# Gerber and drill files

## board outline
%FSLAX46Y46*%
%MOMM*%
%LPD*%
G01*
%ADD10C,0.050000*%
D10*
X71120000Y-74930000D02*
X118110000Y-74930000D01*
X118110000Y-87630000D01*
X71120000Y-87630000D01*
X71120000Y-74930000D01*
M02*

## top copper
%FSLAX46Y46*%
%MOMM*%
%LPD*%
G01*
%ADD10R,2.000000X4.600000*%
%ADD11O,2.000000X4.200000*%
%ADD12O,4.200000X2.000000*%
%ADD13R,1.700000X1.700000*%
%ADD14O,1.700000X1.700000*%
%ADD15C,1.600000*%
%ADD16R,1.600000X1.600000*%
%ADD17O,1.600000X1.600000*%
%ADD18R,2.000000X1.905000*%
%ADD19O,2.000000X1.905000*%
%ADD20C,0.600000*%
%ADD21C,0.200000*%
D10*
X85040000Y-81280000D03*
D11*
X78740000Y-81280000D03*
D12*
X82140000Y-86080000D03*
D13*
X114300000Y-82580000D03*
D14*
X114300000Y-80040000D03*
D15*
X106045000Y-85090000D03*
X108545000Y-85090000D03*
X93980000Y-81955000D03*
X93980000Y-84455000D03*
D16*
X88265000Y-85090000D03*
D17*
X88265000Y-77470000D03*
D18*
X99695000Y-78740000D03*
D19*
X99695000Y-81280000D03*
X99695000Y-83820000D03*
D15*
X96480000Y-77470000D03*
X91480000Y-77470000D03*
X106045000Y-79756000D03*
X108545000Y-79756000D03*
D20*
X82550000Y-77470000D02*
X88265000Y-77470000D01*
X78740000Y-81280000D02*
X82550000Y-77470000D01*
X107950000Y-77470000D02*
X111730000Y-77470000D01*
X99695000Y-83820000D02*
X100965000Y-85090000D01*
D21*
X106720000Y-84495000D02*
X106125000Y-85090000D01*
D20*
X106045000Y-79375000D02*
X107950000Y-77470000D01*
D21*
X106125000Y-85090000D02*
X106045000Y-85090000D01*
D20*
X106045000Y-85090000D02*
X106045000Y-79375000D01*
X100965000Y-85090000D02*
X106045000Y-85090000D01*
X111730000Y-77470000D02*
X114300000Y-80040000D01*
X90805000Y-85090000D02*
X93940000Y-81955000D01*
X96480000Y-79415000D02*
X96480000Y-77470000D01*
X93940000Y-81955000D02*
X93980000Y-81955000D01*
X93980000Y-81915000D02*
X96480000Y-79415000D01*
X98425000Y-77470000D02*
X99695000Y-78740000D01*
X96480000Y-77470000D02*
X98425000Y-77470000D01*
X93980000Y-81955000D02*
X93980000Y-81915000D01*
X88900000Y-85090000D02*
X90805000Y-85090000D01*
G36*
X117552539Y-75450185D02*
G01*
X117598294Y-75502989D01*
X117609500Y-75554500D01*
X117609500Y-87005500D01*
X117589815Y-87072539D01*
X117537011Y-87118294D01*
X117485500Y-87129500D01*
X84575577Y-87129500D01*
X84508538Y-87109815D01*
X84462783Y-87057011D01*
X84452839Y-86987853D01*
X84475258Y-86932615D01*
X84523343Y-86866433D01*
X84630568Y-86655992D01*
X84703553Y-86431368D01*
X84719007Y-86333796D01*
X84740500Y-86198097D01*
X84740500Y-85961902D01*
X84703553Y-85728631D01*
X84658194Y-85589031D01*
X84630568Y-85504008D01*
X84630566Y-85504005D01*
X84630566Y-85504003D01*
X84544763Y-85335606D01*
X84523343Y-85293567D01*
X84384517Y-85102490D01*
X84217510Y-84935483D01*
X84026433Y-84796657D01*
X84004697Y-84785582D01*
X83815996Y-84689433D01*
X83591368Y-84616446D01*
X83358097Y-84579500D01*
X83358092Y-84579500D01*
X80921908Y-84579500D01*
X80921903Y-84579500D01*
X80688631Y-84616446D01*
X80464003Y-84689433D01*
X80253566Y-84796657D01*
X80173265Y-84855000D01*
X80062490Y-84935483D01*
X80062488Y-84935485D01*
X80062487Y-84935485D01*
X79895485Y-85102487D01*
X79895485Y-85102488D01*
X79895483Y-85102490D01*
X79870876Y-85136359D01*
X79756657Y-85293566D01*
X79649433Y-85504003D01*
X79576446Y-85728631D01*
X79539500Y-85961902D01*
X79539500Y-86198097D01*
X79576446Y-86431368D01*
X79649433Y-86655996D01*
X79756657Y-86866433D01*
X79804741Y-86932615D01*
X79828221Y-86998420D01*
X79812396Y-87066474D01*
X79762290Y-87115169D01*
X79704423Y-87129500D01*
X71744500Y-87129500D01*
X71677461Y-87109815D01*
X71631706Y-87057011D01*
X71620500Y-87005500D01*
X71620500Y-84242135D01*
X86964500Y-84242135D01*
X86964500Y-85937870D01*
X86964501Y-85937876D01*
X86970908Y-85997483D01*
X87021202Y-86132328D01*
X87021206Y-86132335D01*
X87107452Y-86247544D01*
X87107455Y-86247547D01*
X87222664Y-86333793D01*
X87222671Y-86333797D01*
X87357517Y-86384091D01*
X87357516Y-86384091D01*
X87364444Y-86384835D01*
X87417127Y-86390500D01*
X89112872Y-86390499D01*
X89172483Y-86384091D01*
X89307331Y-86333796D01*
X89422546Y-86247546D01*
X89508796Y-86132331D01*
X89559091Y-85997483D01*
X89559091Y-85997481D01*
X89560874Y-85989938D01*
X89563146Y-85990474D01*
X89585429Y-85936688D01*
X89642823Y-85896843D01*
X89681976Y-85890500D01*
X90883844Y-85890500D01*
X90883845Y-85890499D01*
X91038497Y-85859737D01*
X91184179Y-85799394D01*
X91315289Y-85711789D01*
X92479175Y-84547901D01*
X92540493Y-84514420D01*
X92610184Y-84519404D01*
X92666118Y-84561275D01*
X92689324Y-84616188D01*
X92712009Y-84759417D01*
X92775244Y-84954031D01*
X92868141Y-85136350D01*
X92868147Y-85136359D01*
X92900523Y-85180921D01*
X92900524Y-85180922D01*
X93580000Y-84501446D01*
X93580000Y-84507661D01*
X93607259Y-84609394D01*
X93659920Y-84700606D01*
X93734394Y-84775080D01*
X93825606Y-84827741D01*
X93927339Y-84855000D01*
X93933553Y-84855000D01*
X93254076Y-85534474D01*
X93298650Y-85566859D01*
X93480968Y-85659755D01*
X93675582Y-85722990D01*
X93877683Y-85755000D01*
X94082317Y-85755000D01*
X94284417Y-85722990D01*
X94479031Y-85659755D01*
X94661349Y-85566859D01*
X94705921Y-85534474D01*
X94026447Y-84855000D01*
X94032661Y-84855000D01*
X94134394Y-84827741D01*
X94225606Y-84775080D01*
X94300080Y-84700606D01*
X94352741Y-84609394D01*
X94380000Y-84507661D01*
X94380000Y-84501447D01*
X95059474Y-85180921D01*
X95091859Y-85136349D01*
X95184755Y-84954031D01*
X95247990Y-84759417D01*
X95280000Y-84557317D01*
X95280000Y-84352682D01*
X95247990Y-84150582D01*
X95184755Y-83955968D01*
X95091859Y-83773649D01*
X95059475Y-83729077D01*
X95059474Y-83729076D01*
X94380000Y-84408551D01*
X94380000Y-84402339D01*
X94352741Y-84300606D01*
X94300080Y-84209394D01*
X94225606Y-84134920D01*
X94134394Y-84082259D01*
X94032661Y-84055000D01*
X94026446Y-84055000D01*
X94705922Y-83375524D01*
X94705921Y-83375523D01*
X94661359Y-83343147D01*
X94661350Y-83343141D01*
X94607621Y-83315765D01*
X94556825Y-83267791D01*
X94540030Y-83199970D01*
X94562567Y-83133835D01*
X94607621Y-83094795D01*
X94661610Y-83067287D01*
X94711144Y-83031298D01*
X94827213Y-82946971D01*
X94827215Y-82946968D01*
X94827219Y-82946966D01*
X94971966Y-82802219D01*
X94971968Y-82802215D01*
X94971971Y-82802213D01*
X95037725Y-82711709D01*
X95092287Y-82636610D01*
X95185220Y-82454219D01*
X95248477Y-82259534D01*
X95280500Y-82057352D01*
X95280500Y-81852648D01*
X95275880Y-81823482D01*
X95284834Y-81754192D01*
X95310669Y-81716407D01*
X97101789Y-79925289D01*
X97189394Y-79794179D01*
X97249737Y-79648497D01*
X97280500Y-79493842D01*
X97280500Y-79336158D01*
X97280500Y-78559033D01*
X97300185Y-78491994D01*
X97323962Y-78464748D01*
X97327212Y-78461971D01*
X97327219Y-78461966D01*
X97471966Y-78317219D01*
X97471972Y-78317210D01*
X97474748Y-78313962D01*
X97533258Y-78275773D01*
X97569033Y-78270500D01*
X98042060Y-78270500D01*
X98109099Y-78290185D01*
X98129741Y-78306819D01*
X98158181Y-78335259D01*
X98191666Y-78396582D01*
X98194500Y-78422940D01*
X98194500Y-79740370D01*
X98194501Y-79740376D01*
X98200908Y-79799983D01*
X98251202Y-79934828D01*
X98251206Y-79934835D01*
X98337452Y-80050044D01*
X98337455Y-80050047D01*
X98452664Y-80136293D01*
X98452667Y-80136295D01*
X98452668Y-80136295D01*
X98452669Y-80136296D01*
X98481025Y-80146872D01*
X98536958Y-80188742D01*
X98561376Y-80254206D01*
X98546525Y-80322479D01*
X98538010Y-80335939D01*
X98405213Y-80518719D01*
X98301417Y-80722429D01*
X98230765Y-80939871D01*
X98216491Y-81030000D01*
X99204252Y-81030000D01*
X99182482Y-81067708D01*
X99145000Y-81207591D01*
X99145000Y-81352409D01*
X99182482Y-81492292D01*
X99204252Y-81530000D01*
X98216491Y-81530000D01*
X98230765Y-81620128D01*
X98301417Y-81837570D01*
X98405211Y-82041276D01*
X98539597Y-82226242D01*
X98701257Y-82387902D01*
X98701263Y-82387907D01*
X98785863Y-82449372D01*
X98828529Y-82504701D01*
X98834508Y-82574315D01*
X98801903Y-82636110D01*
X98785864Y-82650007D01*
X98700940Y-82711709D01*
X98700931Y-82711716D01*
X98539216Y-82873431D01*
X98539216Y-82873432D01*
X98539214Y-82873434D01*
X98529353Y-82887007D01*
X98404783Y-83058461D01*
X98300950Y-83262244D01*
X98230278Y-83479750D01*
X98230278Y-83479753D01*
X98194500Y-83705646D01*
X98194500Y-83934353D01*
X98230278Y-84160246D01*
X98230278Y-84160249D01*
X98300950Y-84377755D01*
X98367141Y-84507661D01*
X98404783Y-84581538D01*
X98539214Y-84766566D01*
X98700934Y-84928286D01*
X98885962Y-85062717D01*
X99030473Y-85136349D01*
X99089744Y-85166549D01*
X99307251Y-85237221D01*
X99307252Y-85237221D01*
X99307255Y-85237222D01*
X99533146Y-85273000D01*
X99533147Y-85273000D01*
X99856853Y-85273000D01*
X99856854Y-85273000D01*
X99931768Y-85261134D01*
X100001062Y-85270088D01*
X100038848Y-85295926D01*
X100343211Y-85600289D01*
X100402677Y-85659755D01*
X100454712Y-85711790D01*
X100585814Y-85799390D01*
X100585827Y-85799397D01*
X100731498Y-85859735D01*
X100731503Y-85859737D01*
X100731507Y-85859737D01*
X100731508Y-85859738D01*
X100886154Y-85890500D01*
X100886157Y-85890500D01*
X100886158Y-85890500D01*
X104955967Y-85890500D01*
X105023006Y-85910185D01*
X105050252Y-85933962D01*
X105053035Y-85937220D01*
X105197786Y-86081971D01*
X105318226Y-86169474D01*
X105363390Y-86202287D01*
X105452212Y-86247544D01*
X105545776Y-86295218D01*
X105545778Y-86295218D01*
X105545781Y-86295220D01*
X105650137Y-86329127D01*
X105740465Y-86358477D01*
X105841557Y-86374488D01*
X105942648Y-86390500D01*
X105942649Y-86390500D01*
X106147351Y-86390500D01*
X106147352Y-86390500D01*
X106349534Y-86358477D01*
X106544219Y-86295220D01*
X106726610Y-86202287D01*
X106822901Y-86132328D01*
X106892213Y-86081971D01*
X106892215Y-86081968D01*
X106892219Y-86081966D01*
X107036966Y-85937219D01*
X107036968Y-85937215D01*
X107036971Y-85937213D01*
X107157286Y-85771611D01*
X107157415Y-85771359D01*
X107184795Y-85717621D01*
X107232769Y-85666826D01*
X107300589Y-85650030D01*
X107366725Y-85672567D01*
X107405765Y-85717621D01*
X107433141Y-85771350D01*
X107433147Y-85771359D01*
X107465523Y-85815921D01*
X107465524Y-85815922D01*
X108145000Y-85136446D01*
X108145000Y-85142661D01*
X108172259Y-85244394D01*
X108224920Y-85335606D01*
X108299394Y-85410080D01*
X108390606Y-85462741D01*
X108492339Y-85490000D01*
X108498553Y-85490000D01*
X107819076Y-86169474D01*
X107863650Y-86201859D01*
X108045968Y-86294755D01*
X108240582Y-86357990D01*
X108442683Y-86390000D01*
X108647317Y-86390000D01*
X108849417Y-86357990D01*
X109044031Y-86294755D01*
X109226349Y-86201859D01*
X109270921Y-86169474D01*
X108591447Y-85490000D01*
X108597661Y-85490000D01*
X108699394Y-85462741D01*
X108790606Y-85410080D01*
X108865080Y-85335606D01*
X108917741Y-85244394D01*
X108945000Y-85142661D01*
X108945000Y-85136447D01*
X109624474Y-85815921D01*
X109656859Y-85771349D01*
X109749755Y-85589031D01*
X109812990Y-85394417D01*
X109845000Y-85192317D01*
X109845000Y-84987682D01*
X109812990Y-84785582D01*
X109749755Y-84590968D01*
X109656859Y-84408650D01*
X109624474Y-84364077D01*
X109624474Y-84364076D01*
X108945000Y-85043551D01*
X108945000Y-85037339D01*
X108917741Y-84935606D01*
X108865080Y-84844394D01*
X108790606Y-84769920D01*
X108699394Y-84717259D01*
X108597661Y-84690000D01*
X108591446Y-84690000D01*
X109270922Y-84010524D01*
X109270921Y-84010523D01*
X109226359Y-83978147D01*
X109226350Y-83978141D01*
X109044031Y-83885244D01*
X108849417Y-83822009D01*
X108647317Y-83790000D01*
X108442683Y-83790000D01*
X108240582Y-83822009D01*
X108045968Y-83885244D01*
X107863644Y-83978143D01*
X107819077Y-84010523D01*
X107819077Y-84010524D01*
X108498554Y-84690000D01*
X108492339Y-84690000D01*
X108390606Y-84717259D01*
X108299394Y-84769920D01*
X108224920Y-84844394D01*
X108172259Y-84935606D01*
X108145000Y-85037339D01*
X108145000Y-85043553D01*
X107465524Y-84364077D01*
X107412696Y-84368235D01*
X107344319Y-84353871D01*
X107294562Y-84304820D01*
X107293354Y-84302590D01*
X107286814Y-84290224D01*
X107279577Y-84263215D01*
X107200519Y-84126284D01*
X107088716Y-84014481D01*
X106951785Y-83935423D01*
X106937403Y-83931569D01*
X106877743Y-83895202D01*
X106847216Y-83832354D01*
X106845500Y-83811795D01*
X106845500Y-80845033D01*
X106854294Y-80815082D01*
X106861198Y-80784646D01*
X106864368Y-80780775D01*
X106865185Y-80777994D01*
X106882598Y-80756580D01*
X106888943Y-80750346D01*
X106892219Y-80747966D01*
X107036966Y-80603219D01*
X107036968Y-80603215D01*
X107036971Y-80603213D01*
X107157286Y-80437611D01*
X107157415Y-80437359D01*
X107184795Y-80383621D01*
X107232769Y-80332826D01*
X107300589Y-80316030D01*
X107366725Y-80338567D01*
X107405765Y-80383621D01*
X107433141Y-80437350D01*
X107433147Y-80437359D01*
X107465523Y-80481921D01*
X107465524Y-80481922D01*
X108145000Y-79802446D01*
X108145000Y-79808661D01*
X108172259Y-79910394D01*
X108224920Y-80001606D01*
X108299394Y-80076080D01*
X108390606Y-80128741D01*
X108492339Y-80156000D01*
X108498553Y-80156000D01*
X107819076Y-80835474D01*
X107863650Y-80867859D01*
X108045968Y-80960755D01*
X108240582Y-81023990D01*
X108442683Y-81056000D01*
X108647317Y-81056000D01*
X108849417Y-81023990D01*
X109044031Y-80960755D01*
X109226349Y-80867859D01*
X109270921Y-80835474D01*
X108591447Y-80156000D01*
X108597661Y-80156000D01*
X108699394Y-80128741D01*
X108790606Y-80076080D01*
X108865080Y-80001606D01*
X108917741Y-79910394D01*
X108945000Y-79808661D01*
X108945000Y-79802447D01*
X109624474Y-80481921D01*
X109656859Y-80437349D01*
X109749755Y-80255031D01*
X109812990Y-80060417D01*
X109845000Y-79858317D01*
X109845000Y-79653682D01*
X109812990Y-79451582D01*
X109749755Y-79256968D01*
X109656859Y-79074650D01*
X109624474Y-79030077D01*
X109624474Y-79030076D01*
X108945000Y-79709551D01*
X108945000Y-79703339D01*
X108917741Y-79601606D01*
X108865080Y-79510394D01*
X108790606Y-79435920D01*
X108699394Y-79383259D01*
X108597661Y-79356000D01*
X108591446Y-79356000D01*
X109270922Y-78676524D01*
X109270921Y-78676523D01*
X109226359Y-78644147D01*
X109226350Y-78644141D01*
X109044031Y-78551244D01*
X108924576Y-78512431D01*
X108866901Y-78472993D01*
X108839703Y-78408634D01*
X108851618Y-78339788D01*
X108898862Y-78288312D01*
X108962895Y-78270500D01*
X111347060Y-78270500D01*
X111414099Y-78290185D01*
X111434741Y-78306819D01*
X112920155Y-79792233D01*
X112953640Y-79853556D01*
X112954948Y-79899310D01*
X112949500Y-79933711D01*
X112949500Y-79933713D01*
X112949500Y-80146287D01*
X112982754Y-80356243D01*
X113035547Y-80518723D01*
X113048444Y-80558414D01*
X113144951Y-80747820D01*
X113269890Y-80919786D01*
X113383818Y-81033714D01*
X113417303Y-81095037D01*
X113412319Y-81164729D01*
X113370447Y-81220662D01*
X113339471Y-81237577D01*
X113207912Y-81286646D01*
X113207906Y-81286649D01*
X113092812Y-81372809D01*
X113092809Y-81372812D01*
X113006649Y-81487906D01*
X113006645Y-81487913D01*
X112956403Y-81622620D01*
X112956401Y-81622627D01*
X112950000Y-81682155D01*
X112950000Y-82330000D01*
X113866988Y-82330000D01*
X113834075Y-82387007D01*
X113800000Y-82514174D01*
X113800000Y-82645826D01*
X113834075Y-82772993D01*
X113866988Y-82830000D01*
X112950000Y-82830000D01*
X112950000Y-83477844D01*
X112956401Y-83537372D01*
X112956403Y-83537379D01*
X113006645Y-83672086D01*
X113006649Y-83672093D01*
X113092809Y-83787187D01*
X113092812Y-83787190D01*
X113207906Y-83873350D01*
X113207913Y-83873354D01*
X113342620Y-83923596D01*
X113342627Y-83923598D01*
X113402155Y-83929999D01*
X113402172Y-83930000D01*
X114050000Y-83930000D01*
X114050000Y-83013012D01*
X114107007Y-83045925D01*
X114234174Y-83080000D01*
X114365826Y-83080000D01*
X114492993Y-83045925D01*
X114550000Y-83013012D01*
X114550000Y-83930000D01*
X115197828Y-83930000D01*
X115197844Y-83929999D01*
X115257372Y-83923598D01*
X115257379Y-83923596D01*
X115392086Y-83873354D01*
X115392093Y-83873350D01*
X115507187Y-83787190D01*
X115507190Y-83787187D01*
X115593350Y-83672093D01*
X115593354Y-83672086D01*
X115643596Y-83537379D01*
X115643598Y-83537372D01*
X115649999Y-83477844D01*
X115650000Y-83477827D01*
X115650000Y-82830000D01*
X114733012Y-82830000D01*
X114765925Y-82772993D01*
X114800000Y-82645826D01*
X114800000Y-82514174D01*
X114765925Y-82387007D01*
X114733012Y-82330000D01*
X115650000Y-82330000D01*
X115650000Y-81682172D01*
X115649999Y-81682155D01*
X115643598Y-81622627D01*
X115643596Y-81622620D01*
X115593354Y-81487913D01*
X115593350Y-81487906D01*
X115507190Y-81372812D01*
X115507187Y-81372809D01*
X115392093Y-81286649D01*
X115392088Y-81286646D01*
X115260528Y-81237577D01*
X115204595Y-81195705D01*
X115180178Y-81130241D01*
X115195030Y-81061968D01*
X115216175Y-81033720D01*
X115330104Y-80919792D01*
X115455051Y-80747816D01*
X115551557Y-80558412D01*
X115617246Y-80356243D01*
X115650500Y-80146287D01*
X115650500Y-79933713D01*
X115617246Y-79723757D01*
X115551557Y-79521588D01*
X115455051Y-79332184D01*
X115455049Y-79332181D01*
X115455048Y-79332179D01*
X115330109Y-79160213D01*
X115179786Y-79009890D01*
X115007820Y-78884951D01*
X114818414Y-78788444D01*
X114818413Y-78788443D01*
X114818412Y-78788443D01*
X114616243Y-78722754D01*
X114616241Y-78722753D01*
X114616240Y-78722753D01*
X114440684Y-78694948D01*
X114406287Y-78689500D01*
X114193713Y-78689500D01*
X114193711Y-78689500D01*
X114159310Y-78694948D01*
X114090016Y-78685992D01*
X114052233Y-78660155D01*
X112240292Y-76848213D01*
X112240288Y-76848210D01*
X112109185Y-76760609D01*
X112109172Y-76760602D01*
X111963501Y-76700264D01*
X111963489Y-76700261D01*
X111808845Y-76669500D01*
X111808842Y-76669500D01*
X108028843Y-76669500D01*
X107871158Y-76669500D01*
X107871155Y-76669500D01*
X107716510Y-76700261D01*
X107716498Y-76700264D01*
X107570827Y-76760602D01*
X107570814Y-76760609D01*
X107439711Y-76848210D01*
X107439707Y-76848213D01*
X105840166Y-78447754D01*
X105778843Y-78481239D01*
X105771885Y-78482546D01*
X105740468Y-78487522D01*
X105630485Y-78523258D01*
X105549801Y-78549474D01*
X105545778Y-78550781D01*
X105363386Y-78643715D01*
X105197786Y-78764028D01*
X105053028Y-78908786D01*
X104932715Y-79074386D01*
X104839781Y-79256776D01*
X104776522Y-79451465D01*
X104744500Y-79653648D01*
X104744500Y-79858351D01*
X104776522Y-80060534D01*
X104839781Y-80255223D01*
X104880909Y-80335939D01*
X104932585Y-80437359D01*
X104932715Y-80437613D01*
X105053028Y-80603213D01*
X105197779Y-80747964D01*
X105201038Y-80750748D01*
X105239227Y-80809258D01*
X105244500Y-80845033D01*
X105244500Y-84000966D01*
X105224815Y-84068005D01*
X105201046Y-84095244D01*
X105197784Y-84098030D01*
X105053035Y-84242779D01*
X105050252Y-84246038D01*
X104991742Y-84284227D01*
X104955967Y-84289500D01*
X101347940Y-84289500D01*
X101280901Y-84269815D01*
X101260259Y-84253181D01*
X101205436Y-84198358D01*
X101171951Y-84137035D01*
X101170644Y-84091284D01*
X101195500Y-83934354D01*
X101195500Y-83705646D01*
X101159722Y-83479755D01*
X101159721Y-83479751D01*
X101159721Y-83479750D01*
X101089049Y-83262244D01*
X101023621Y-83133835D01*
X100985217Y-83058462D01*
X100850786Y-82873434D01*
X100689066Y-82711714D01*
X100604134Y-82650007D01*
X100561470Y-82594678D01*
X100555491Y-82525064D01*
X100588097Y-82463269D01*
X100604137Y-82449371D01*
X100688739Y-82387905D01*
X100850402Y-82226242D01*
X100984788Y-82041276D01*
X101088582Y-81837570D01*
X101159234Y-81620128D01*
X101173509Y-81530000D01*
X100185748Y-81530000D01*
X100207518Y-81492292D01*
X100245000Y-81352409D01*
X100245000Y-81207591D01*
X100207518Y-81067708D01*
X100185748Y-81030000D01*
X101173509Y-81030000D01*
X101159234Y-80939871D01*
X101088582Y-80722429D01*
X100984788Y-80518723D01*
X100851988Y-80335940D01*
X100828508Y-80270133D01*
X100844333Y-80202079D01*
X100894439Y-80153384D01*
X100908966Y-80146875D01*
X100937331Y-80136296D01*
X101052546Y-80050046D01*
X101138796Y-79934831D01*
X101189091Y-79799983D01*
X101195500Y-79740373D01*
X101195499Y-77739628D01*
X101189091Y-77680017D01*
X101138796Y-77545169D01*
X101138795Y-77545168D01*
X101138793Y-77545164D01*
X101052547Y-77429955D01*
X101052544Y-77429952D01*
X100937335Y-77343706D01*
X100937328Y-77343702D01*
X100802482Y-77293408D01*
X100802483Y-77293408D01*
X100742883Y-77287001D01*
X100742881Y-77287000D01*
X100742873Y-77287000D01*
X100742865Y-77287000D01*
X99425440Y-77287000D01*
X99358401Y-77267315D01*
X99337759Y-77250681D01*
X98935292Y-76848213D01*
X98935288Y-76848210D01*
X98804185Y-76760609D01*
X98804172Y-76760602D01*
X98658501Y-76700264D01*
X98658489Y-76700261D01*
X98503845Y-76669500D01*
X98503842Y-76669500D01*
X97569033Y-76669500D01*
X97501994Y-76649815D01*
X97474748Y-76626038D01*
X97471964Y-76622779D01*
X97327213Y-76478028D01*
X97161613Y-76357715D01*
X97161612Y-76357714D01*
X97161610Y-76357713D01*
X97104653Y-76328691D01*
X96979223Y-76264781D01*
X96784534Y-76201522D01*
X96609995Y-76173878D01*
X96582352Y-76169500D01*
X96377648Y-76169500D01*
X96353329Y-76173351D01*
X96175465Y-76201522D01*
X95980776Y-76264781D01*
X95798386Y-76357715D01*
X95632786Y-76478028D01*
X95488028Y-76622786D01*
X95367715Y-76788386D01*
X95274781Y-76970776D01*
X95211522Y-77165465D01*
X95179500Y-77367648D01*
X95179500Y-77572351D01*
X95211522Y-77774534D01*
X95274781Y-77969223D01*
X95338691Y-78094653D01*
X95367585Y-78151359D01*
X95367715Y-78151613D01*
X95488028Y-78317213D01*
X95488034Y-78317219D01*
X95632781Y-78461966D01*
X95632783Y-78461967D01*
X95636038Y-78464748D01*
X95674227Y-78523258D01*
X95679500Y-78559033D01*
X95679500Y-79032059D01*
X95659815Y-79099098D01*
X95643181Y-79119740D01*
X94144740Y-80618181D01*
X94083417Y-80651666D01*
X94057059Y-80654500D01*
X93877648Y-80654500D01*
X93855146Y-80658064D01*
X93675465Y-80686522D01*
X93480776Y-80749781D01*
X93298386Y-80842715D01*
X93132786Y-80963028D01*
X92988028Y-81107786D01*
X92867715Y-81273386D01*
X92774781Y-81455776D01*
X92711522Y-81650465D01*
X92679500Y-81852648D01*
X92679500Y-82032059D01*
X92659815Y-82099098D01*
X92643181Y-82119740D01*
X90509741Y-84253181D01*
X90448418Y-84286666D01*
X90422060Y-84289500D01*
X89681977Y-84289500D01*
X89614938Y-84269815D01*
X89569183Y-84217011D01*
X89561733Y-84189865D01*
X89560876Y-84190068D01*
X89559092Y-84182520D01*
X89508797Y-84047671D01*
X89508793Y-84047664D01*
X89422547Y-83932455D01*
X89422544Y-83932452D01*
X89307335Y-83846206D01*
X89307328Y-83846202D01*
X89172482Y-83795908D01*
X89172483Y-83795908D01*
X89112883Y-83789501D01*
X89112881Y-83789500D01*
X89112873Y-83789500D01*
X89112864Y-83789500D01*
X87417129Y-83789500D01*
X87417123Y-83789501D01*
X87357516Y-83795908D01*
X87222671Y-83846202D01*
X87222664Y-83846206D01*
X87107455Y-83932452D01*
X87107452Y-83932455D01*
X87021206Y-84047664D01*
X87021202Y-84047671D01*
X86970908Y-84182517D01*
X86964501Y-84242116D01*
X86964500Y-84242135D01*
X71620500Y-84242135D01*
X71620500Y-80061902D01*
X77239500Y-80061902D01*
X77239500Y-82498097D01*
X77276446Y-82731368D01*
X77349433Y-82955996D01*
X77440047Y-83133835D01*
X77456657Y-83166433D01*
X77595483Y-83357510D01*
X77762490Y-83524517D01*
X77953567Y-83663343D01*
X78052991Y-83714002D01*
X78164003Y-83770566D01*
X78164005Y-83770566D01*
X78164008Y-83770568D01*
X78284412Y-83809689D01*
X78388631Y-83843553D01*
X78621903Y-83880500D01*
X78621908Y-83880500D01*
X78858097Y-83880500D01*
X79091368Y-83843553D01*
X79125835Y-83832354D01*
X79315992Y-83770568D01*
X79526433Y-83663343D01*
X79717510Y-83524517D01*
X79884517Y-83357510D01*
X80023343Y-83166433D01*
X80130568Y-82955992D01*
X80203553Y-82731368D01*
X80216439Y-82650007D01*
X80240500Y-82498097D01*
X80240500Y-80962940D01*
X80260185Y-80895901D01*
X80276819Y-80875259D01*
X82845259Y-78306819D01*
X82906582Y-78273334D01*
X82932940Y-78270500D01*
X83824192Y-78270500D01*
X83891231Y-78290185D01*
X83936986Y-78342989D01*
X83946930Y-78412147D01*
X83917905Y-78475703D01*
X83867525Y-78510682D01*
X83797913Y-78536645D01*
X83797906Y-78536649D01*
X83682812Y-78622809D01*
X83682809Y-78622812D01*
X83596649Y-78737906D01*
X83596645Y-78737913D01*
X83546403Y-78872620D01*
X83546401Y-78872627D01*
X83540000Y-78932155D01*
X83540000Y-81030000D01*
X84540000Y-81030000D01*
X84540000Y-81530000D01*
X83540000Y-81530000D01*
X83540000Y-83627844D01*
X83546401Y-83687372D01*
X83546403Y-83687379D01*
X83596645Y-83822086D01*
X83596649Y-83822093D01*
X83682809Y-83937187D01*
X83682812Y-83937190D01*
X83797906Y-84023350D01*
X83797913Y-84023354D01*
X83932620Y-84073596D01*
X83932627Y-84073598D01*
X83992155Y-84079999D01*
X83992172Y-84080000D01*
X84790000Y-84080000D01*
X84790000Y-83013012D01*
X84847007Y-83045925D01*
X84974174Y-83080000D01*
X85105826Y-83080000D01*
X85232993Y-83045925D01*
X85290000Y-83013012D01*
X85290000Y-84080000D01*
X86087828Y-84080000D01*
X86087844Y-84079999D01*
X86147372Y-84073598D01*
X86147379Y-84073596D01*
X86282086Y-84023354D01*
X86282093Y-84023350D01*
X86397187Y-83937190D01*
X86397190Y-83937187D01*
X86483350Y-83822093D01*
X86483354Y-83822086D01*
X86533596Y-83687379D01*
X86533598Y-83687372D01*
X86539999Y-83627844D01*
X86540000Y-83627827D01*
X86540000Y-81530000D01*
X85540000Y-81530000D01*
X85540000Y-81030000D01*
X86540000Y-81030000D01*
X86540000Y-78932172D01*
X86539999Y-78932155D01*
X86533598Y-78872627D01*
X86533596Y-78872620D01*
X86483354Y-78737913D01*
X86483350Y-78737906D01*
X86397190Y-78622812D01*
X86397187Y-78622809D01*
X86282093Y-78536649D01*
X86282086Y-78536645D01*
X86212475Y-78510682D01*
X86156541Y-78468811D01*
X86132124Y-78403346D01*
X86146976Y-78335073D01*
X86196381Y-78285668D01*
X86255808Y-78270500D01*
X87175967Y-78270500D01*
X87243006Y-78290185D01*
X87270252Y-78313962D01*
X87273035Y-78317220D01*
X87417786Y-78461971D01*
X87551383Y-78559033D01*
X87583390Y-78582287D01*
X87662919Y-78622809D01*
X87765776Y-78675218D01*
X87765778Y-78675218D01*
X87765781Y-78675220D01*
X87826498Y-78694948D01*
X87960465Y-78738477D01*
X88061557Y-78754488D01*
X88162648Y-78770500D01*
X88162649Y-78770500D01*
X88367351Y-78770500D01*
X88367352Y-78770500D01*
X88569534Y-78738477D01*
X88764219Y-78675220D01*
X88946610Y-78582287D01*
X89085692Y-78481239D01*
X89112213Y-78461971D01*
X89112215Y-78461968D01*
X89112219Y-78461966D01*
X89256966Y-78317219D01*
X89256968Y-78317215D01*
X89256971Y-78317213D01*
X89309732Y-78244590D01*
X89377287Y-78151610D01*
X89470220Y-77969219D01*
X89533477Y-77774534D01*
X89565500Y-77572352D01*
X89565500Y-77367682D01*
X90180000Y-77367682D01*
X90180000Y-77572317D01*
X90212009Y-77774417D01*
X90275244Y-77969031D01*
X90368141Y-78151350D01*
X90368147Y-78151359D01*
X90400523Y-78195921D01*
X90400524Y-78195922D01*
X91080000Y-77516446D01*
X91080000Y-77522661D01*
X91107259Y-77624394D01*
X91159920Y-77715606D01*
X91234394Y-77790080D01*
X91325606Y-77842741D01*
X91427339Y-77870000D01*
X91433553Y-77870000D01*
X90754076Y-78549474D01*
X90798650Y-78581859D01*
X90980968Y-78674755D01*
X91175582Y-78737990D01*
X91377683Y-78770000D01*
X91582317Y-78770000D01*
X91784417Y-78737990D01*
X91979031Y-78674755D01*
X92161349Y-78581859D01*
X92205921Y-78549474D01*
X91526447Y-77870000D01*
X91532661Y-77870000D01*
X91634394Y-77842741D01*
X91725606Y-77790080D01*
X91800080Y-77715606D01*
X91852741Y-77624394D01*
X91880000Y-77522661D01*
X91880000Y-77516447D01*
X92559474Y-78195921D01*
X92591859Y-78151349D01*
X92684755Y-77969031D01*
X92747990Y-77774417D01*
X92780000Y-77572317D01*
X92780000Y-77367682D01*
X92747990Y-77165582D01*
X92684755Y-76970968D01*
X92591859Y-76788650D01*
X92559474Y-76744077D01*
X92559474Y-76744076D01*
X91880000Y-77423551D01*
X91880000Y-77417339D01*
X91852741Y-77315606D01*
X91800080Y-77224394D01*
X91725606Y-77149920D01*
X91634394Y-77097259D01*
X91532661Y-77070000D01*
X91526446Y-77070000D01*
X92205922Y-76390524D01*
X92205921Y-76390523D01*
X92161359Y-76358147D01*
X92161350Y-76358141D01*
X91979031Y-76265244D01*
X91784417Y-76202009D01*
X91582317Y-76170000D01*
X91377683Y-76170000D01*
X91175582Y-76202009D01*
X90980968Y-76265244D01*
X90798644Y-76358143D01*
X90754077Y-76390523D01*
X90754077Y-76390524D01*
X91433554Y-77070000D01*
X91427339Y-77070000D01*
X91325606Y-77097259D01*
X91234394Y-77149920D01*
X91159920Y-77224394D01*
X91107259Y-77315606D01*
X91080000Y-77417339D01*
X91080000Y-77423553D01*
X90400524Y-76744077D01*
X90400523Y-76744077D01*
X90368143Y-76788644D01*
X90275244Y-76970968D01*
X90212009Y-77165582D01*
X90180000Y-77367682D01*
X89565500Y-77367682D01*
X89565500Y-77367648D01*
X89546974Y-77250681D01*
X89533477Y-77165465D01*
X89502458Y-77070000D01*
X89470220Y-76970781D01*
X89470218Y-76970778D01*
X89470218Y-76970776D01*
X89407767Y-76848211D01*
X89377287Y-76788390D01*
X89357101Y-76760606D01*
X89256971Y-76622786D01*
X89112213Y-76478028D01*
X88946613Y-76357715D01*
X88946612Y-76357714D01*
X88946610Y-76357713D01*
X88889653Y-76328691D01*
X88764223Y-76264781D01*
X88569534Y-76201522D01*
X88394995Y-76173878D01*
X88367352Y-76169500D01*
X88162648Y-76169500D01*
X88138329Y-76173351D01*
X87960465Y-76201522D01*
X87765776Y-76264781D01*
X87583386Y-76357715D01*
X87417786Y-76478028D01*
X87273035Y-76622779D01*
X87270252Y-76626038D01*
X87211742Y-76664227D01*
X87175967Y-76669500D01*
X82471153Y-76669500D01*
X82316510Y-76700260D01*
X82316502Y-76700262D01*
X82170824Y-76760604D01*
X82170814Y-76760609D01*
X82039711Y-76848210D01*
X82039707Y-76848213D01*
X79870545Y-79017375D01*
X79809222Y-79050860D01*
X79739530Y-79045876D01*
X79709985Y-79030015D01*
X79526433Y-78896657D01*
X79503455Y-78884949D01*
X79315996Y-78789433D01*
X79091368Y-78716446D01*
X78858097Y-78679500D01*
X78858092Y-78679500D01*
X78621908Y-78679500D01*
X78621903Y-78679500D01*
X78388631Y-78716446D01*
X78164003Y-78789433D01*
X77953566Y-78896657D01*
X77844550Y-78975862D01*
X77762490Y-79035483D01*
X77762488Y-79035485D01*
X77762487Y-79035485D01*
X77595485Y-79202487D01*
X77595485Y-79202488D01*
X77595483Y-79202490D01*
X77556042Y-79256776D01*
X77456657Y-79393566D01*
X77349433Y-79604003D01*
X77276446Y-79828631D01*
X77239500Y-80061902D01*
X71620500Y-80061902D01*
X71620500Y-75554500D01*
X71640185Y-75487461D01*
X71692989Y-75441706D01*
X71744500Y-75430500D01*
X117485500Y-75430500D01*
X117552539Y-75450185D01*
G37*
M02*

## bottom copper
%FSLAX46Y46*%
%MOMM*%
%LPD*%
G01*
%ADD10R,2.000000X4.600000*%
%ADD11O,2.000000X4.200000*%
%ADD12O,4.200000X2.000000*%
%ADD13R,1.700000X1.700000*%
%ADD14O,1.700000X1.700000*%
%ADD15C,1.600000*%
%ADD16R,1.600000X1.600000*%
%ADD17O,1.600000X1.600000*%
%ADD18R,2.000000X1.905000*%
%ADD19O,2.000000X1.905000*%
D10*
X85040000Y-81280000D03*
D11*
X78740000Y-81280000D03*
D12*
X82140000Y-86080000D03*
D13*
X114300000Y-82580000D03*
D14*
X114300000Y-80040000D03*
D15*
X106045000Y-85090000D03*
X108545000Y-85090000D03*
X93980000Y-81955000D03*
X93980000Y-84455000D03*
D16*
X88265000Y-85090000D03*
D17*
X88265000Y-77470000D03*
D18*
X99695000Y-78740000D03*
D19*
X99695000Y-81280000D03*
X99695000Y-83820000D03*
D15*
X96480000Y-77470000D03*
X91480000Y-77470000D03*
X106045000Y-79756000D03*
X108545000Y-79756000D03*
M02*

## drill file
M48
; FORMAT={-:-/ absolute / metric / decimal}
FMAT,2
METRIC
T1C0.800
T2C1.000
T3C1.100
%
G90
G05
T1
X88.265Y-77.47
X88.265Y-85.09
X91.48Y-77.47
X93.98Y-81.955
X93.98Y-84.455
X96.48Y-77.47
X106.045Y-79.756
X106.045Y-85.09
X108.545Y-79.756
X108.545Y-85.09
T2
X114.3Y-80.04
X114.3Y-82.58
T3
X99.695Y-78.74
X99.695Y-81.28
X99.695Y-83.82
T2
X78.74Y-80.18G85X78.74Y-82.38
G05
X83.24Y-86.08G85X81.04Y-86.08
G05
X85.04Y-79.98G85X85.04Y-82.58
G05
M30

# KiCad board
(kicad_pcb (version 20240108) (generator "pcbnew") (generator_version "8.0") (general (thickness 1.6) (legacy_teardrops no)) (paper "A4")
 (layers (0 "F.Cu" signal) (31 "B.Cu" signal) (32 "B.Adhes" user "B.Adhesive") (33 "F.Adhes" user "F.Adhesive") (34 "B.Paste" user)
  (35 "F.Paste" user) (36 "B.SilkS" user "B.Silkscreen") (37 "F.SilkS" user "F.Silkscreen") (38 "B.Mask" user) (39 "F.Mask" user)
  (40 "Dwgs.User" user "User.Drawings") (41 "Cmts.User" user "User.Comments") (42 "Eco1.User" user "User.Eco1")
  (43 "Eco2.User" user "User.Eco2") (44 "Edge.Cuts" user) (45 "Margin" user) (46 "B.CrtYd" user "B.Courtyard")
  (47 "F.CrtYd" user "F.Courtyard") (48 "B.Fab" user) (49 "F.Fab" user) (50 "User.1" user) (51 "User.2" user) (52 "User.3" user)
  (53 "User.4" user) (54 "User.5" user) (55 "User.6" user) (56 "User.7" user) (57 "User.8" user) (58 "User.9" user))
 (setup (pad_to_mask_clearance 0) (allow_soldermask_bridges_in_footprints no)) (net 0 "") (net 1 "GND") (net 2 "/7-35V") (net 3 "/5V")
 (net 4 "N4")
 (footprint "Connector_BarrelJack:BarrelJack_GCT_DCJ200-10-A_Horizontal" (layer "F.Cu") (at 85.04 81.28 -90)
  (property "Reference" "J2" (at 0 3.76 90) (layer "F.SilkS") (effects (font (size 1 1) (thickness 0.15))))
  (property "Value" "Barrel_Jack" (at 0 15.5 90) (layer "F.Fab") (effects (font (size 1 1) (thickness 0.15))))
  (pad "1" thru_hole rect (at 0 0 270) (size 4.6 2) (drill oval 3.6 1) (layers "*.Cu" "*.Mask") (remove_unused_layers no) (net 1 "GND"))
  (pad "2" thru_hole oval (at 0 6.3 270) (size 4.2 2) (drill oval 3.2 1) (layers "*.Cu" "*.Mask") (remove_unused_layers no) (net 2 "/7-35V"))
  (pad "3" thru_hole oval (at 4.8 2.9 270) (size 2 4.2) (drill oval 1 3.2) (layers "*.Cu" "*.Mask") (remove_unused_layers no)))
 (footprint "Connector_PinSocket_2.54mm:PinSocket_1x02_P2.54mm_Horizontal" (layer "F.Cu") (at 114.3 82.58 180)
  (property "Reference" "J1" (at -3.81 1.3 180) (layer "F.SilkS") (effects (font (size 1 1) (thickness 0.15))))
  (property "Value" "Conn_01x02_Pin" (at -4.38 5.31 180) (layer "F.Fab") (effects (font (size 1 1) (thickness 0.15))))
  (pad "1" thru_hole rect (at 0 0 180) (size 1.7 1.7) (drill 1) (layers "*.Cu" "*.Mask") (remove_unused_layers no) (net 1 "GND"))
  (pad "2" thru_hole oval (at 0 2.54 180) (size 1.7 1.7) (drill 1) (layers "*.Cu" "*.Mask") (remove_unused_layers no) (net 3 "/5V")))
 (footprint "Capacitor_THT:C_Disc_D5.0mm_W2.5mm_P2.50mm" (layer "F.Cu") (at 106.045 85.09)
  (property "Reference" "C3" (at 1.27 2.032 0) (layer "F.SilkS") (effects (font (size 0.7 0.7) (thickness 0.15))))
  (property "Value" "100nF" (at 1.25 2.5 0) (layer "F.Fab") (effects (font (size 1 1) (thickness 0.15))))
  (pad "1" thru_hole circle (at 0 0) (size 1.6 1.6) (drill 0.8) (layers "*.Cu" "*.Mask") (remove_unused_layers no) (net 3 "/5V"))
  (pad "2" thru_hole circle (at 2.5 0) (size 1.6 1.6) (drill 0.8) (layers "*.Cu" "*.Mask") (remove_unused_layers no) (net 1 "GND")))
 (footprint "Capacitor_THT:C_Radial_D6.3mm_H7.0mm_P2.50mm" (layer "F.Cu") (at 93.98 81.955 -90)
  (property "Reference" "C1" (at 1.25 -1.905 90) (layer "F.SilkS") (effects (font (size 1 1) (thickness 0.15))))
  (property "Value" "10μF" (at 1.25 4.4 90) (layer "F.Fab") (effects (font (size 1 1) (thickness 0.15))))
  (pad "1" thru_hole circle (at 0 0 270) (size 1.6 1.6) (drill 0.8) (layers "*.Cu" "*.Mask") (remove_unused_layers no) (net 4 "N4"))
  (pad "2" thru_hole circle (at 2.5 0 270) (size 1.6 1.6) (drill 0.8) (layers "*.Cu" "*.Mask") (remove_unused_layers no) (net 1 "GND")))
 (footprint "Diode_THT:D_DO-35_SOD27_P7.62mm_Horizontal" (layer "F.Cu") (at 88.265 85.09 90)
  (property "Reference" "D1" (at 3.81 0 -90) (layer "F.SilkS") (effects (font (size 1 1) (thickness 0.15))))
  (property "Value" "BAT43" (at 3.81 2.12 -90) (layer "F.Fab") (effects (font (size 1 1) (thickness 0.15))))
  (pad "1" thru_hole rect (at 0 0 90) (size 1.6 1.6) (drill 0.8) (layers "*.Cu" "*.Mask") (remove_unused_layers no) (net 4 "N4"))
  (pad "2" thru_hole oval (at 7.62 0 90) (size 1.6 1.6) (drill 0.8) (layers "*.Cu" "*.Mask") (remove_unused_layers no) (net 2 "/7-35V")))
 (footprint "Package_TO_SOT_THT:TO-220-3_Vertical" (layer "F.Cu") (at 99.695 78.74 -90)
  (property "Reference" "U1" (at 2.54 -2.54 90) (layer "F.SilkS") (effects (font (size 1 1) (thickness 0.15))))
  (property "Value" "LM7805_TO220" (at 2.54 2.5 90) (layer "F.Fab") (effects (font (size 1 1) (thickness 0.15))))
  (pad "1" thru_hole rect (at 0 0 270) (size 1.905 2) (drill 1.1) (layers "*.Cu" "*.Mask") (remove_unused_layers no) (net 4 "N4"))
  (pad "2" thru_hole oval (at 2.54 0 270) (size 1.905 2) (drill 1.1) (layers "*.Cu" "*.Mask") (remove_unused_layers no) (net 1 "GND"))
  (pad "3" thru_hole oval (at 5.08 0 270) (size 1.905 2) (drill 1.1) (layers "*.Cu" "*.Mask") (remove_unused_layers no) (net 3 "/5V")))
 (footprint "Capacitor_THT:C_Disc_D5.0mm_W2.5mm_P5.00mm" (layer "F.Cu") (at 96.48 77.47 180)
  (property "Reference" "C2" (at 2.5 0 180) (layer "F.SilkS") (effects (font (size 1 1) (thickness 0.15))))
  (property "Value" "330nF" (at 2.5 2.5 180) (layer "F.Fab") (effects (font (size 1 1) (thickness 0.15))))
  (pad "1" thru_hole circle (at 0 0 180) (size 1.6 1.6) (drill 0.8) (layers "*.Cu" "*.Mask") (remove_unused_layers no) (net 4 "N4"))
  (pad "2" thru_hole circle (at 5 0 180) (size 1.6 1.6) (drill 0.8) (layers "*.Cu" "*.Mask") (remove_unused_layers no) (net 1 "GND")))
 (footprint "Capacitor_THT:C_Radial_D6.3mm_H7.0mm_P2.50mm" (layer "F.Cu") (at 106.045 79.756)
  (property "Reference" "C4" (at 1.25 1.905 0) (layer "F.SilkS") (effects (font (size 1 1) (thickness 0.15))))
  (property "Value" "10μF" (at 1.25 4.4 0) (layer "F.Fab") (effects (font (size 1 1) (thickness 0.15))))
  (pad "1" thru_hole circle (at 0 0) (size 1.6 1.6) (drill 0.8) (layers "*.Cu" "*.Mask") (remove_unused_layers no) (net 3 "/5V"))
  (pad "2" thru_hole circle (at 2.5 0) (size 1.6 1.6) (drill 0.8) (layers "*.Cu" "*.Mask") (remove_unused_layers no) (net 1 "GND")))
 (gr_rect (start 71.12 74.93) (end 118.11 87.63) (stroke (width 0.05) (type default)) (fill none) (layer "Edge.Cuts"))
 (segment (start 82.55 77.47) (end 88.265 77.47) (width 0.6) (layer "F.Cu") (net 2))
 (segment (start 78.74 81.28) (end 82.55 77.47) (width 0.6) (layer "F.Cu") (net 2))
 (segment (start 107.95 77.47) (end 111.73 77.47) (width 0.6) (layer "F.Cu") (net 3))
 (segment (start 99.695 83.82) (end 100.965 85.09) (width 0.6) (layer "F.Cu") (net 3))
 (segment (start 106.72 84.495) (end 106.125 85.09) (width 0.2) (layer "F.Cu") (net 3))
 (segment (start 106.045 79.375) (end 107.95 77.47) (width 0.6) (layer "F.Cu") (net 3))
 (segment (start 106.125 85.09) (end 106.045 85.09) (width 0.2) (layer "F.Cu") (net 3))
 (segment (start 106.045 85.09) (end 106.045 79.375) (width 0.6) (layer "F.Cu") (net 3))
 (segment (start 100.965 85.09) (end 106.045 85.09) (width 0.6) (layer "F.Cu") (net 3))
 (segment (start 111.73 77.47) (end 114.3 80.04) (width 0.6) (layer "F.Cu") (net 3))
 (segment (start 90.805 85.09) (end 93.94 81.955) (width 0.6) (layer "F.Cu") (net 4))
 (segment (start 96.48 79.415) (end 96.48 77.47) (width 0.6) (layer "F.Cu") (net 4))
 (segment (start 93.94 81.955) (end 93.98 81.955) (width 0.6) (layer "F.Cu") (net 4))
 (segment (start 93.98 81.915) (end 96.48 79.415) (width 0.6) (layer "F.Cu") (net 4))
 (segment (start 98.425 77.47) (end 99.695 78.74) (width 0.6) (layer "F.Cu") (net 4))
 (segment (start 96.48 77.47) (end 98.425 77.47) (width 0.6) (layer "F.Cu") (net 4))
 (segment (start 93.98 81.955) (end 93.98 81.915) (width 0.6) (layer "F.Cu") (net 4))
 (segment (start 88.9 85.09) (end 90.805 85.09) (width 0.6) (layer "F.Cu") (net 4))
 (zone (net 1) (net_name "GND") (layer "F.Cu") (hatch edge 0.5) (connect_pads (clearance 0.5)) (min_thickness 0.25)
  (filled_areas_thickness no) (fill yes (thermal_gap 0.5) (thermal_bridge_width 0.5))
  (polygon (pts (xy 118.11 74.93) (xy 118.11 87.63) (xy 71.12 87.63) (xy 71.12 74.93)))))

